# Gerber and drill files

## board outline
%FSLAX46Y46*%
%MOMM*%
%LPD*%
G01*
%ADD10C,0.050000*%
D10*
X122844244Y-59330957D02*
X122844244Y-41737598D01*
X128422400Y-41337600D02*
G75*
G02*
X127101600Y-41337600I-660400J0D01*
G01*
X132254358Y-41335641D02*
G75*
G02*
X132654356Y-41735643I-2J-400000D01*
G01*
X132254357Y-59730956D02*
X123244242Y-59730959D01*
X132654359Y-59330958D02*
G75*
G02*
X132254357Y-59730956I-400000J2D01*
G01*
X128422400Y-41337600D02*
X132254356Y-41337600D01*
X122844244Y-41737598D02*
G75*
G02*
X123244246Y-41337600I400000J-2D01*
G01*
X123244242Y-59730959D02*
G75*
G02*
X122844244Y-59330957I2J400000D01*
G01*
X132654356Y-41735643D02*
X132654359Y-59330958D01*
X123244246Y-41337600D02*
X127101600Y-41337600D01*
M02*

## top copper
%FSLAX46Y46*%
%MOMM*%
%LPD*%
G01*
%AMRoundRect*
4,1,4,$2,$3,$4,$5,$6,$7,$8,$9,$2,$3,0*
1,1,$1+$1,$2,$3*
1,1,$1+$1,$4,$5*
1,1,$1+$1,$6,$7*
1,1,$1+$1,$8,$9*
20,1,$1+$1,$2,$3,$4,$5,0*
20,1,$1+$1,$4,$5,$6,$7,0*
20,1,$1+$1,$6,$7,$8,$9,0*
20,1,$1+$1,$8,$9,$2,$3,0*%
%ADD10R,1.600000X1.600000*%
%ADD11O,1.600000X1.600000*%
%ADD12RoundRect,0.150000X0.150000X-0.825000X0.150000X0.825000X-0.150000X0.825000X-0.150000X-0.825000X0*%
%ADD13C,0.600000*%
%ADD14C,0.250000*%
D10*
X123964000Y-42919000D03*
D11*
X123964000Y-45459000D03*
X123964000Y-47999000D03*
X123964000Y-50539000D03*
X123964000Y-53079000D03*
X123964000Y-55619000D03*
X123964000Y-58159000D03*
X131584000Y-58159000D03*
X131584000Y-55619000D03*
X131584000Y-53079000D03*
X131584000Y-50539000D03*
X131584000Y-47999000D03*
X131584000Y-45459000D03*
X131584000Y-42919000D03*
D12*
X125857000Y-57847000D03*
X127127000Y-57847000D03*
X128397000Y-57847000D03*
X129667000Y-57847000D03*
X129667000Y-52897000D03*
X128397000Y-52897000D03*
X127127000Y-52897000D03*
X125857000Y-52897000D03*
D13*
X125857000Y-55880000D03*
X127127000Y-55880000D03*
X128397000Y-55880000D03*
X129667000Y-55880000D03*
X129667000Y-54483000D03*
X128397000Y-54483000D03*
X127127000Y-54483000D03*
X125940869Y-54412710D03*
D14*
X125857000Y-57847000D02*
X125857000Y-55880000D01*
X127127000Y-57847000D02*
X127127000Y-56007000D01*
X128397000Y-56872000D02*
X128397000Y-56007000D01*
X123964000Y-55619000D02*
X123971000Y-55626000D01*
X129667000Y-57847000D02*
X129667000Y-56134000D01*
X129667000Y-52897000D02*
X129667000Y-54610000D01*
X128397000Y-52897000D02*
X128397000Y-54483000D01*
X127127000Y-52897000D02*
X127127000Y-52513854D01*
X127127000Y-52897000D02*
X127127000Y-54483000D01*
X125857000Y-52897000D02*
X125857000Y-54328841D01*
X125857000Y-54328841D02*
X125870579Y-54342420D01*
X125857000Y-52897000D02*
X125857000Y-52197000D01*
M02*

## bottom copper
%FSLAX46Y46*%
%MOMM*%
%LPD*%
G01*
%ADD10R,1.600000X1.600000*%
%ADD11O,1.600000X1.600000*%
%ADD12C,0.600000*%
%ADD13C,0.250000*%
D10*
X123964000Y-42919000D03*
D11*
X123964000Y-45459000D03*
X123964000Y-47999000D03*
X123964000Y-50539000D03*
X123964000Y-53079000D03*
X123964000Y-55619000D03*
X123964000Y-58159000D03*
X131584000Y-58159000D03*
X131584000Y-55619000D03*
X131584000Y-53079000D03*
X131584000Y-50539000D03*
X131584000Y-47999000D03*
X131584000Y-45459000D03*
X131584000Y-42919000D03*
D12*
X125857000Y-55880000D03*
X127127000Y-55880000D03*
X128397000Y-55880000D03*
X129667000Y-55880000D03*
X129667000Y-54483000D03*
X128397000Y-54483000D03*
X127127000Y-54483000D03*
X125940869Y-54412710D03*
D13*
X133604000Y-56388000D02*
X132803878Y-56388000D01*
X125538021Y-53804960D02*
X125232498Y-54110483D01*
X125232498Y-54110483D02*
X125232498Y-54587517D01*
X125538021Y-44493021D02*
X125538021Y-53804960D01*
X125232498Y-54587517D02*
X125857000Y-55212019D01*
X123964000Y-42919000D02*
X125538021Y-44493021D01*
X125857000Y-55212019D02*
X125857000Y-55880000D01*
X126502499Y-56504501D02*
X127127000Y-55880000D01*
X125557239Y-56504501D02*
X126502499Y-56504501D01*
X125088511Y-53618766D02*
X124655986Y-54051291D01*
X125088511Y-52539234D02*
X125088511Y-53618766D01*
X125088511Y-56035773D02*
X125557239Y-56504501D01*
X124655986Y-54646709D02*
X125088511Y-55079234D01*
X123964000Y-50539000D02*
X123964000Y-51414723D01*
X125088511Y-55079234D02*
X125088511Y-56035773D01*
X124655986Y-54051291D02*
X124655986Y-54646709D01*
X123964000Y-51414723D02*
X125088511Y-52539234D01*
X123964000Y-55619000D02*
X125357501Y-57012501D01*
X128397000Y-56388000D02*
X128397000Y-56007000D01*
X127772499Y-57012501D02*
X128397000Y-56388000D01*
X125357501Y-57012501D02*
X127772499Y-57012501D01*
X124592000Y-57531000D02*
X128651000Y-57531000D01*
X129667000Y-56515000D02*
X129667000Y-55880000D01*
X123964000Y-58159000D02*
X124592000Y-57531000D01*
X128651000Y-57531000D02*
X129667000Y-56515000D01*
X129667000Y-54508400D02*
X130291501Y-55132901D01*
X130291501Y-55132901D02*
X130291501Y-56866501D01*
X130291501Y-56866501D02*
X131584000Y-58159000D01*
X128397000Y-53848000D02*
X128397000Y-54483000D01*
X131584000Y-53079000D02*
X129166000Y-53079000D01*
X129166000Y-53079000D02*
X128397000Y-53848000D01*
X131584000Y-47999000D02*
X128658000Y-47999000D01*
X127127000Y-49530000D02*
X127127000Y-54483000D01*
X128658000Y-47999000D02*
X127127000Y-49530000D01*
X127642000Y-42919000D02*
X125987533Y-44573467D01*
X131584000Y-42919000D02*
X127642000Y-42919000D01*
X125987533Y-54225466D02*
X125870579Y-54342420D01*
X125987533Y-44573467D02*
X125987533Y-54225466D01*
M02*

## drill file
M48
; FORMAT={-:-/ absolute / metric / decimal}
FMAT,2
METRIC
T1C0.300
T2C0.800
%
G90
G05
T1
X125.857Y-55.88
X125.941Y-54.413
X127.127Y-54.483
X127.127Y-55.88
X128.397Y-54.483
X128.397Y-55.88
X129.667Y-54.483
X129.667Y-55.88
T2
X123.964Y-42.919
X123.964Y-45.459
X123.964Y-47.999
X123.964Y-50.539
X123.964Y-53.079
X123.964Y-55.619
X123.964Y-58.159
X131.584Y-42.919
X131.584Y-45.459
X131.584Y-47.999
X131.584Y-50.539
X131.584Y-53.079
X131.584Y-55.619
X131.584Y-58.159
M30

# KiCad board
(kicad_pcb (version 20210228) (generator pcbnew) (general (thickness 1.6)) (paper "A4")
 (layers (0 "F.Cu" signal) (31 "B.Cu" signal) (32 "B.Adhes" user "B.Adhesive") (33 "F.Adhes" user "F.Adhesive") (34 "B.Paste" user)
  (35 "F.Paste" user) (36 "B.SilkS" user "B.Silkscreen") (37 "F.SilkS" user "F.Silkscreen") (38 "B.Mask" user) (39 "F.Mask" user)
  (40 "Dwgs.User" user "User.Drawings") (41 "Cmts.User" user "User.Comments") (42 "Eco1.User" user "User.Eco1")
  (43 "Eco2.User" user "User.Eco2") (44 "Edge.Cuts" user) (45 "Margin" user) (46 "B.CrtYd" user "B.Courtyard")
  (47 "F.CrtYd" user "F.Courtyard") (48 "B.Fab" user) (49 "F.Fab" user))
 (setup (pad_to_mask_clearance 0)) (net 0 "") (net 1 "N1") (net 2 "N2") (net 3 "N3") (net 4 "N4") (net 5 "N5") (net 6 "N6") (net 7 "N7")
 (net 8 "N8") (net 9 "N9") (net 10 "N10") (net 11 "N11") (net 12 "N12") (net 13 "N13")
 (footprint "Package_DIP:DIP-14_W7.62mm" (layer "F.Cu") (at 123.964 42.919)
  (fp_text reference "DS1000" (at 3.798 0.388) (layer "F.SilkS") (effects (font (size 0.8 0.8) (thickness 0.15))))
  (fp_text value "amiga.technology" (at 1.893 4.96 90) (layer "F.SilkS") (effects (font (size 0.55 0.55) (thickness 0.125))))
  (pad "1" thru_hole rect (at 0 0) (locked) (size 1.6 1.6) (drill 0.8) (layers *.Cu *.Mask) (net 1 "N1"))
  (pad "2" thru_hole oval (at 0 2.54) (locked) (size 1.6 1.6) (drill 0.8) (layers *.Cu *.Mask) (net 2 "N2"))
  (pad "3" thru_hole oval (at 0 5.08) (locked) (size 1.6 1.6) (drill 0.8) (layers *.Cu *.Mask) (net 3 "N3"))
  (pad "4" thru_hole oval (at 0 7.62) (locked) (size 1.6 1.6) (drill 0.8) (layers *.Cu *.Mask) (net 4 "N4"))
  (pad "5" thru_hole oval (at 0 10.16) (locked) (size 1.6 1.6) (drill 0.8) (layers *.Cu *.Mask))
  (pad "6" thru_hole oval (at 0 12.7) (locked) (size 1.6 1.6) (drill 0.8) (layers *.Cu *.Mask) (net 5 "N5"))
  (pad "7" thru_hole oval (at 0 15.24) (locked) (size 1.6 1.6) (drill 0.8) (layers *.Cu *.Mask) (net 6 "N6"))
  (pad "8" thru_hole oval (at 7.62 15.24) (locked) (size 1.6 1.6) (drill 0.8) (layers *.Cu *.Mask) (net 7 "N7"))
  (pad "9" thru_hole oval (at 7.62 12.7) (locked) (size 1.6 1.6) (drill 0.8) (layers *.Cu *.Mask) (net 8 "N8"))
  (pad "10" thru_hole oval (at 7.62 10.16) (locked) (size 1.6 1.6) (drill 0.8) (layers *.Cu *.Mask) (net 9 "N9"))
  (pad "11" thru_hole oval (at 7.62 7.62) (locked) (size 1.6 1.6) (drill 0.8) (layers *.Cu *.Mask) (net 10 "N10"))
  (pad "12" thru_hole oval (at 7.62 5.08) (locked) (size 1.6 1.6) (drill 0.8) (layers *.Cu *.Mask) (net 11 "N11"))
  (pad "13" thru_hole oval (at 7.62 2.54) (locked) (size 1.6 1.6) (drill 0.8) (layers *.Cu *.Mask) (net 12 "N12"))
  (pad "14" thru_hole oval (at 7.62 0) (locked) (size 1.6 1.6) (drill 0.8) (layers *.Cu *.Mask) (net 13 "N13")))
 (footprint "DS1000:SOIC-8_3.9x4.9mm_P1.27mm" (layer "F.Cu") (at 127.762 55.372 90)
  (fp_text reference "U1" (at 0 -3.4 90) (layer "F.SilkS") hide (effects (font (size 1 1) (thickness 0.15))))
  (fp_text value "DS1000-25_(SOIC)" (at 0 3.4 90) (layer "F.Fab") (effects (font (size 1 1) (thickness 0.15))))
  (pad "1" smd roundrect (at -2.475 -1.905 90) (locked) (size 1.95 0.6) (layers "F.Cu" "F.Paste" "F.Mask") (roundrect_rratio 0.25)
   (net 1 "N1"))
  (pad "2" smd roundrect (at -2.475 -0.635 90) (locked) (size 1.95 0.6) (layers "F.Cu" "F.Paste" "F.Mask") (roundrect_rratio 0.25)
   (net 4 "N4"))
  (pad "3" smd roundrect (at -2.475 0.635 90) (locked) (size 1.95 0.6) (layers "F.Cu" "F.Paste" "F.Mask") (roundrect_rratio 0.25)
   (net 5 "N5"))
  (pad "4" smd roundrect (at -2.475 1.905 90) (locked) (size 1.95 0.6) (layers "F.Cu" "F.Paste" "F.Mask") (roundrect_rratio 0.25)
   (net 6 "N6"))
  (pad "5" smd roundrect (at 2.475 1.905 90) (locked) (size 1.95 0.6) (layers "F.Cu" "F.Paste" "F.Mask") (roundrect_rratio 0.25)
   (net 7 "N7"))
  (pad "6" smd roundrect (at 2.475 0.635 90) (locked) (size 1.95 0.6) (layers "F.Cu" "F.Paste" "F.Mask") (roundrect_rratio 0.25)
   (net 9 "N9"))
  (pad "7" smd roundrect (at 2.475 -0.635 90) (locked) (size 1.95 0.6) (layers "F.Cu" "F.Paste" "F.Mask") (roundrect_rratio 0.25)
   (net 11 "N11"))
  (pad "8" smd roundrect (at 2.475 -1.905 90) (locked) (size 1.95 0.6) (layers "F.Cu" "F.Paste" "F.Mask") (roundrect_rratio 0.25)
   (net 13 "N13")))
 (gr_line (start 122.844244 59.330957) (end 122.844244 41.737598) (layer "Edge.Cuts") (width 0.05))
 (gr_arc (start 127.762 41.3376) (end 128.4224 41.3376) (angle 180) (layer "Edge.Cuts") (width 0.05))
 (gr_arc (start 132.254356 41.735641) (end 132.654356 41.735643) (angle -90) (layer "Edge.Cuts") (width 0.05))
 (gr_line (start 132.254357 59.730956) (end 123.244242 59.730959) (layer "Edge.Cuts") (width 0.05))
 (gr_arc (start 132.254359 59.330956) (end 132.254357 59.730956) (angle -90) (layer "Edge.Cuts") (width 0.05))
 (gr_line (start 128.4224 41.3376) (end 132.254356 41.3376) (layer "Edge.Cuts") (width 0.05))
 (gr_arc (start 123.244244 41.7376) (end 123.244246 41.3376) (angle -90) (layer "Edge.Cuts") (width 0.05))
 (gr_arc (start 123.244244 59.330959) (end 122.844244 59.330957) (angle -90) (layer "Edge.Cuts") (width 0.05))
 (gr_line (start 132.654356 41.735643) (end 132.654359 59.330958) (layer "Edge.Cuts") (width 0.05))
 (gr_line (start 123.244246 41.3376) (end 127.1016 41.3376) (layer "Edge.Cuts") (width 0.05))
 (segment (start 133.604 56.388) (end 132.803878 56.388) (width 0.25) (layer "B.Cu") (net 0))
 (segment (start 125.857 57.847) (end 125.857 55.88) (width 0.25) (layer "F.Cu") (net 1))
 (via (at 125.857 55.88) (size 0.6) (drill 0.3) (layers "F.Cu" "B.Cu") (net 1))
 (segment (start 125.538021 53.80496) (end 125.232498 54.110483) (width 0.25) (layer "B.Cu") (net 1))
 (segment (start 125.232498 54.110483) (end 125.232498 54.587517) (width 0.25) (layer "B.Cu") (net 1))
 (segment (start 125.538021 44.493021) (end 125.538021 53.80496) (width 0.25) (layer "B.Cu") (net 1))
 (segment (start 125.232498 54.587517) (end 125.857 55.212019) (width 0.25) (layer "B.Cu") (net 1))
 (segment (start 123.964 42.919) (end 125.538021 44.493021) (width 0.25) (layer "B.Cu") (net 1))
 (segment (start 125.857 55.212019) (end 125.857 55.88) (width 0.25) (layer "B.Cu") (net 1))
 (segment (start 127.127 57.847) (end 127.127 56.007) (width 0.25) (layer "F.Cu") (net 4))
 (via (at 127.127 55.88) (size 0.6) (drill 0.3) (layers "F.Cu" "B.Cu") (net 4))
 (segment (start 126.502499 56.504501) (end 127.127 55.88) (width 0.25) (layer "B.Cu") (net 4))
 (segment (start 125.557239 56.504501) (end 126.502499 56.504501) (width 0.25) (layer "B.Cu") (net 4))
 (segment (start 125.088511 53.618766) (end 124.655986 54.051291) (width 0.25) (layer "B.Cu") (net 4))
 (segment (start 125.088511 52.539234) (end 125.088511 53.618766) (width 0.25) (layer "B.Cu") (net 4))
 (segment (start 125.088511 56.035773) (end 125.557239 56.504501) (width 0.25) (layer "B.Cu") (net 4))
 (segment (start 124.655986 54.646709) (end 125.088511 55.079234) (width 0.25) (layer "B.Cu") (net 4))
 (segment (start 123.964 50.539) (end 123.964 51.414723) (width 0.25) (layer "B.Cu") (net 4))
 (segment (start 125.088511 55.079234) (end 125.088511 56.035773) (width 0.25) (layer "B.Cu") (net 4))
 (segment (start 124.655986 54.051291) (end 124.655986 54.646709) (width 0.25) (layer "B.Cu") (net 4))
 (segment (start 123.964 51.414723) (end 125.088511 52.539234) (width 0.25) (layer "B.Cu") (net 4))
 (segment (start 128.397 56.872) (end 128.397 56.007) (width 0.25) (layer "F.Cu") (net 5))
 (segment (start 123.964 55.619) (end 123.971 55.626) (width 0.25) (layer "F.Cu") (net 5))
 (via (at 128.397 55.88) (size 0.6) (drill 0.3) (layers "F.Cu" "B.Cu") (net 5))
 (segment (start 123.964 55.619) (end 125.357501 57.012501) (width 0.25) (layer "B.Cu") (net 5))
 (segment (start 128.397 56.388) (end 128.397 56.007) (width 0.25) (layer "B.Cu") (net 5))
 (segment (start 127.772499 57.012501) (end 128.397 56.388) (width 0.25) (layer "B.Cu") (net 5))
 (segment (start 125.357501 57.012501) (end 127.772499 57.012501) (width 0.25) (layer "B.Cu") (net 5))
 (segment (start 129.667 57.847) (end 129.667 56.134) (width 0.25) (layer "F.Cu") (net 6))
 (via (at 129.667 55.88) (size 0.6) (drill 0.3) (layers "F.Cu" "B.Cu") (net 6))
 (segment (start 124.592 57.531) (end 128.651 57.531) (width 0.25) (layer "B.Cu") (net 6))
 (segment (start 129.667 56.515) (end 129.667 55.88) (width 0.25) (layer "B.Cu") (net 6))
 (segment (start 123.964 58.159) (end 124.592 57.531) (width 0.25) (layer "B.Cu") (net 6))
 (segment (start 128.651 57.531) (end 129.667 56.515) (width 0.25) (layer "B.Cu") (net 6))
 (segment (start 129.667 52.897) (end 129.667 54.61) (width 0.25) (layer "F.Cu") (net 7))
 (via (at 129.667 54.483) (size 0.6) (drill 0.3) (layers "F.Cu" "B.Cu") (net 7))
 (segment (start 129.667 54.5084) (end 130.291501 55.132901) (width 0.25) (layer "B.Cu") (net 7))
 (segment (start 130.291501 55.132901) (end 130.291501 56.866501) (width 0.25) (layer "B.Cu") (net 7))
 (segment (start 130.291501 56.866501) (end 131.584 58.159) (width 0.25) (layer "B.Cu") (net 7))
 (segment (start 128.397 52.897) (end 128.397 54.483) (width 0.25) (layer "F.Cu") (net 9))
 (via (at 128.397 54.483) (size 0.6) (drill 0.3) (layers "F.Cu" "B.Cu") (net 9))
 (segment (start 128.397 53.848) (end 128.397 54.483) (width 0.25) (layer "B.Cu") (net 9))
 (segment (start 131.584 53.079) (end 129.166 53.079) (width 0.25) (layer "B.Cu") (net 9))
 (segment (start 129.166 53.079) (end 128.397 53.848) (width 0.25) (layer "B.Cu") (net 9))
 (segment (start 127.127 52.897) (end 127.127 52.513854) (width 0.25) (layer "F.Cu") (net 11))
 (segment (start 127.127 52.897) (end 127.127 54.483) (width 0.25) (layer "F.Cu") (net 11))
 (via (at 127.127 54.483) (size 0.6) (drill 0.3) (layers "F.Cu" "B.Cu") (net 11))
 (segment (start 131.584 47.999) (end 128.658 47.999) (width 0.25) (layer "B.Cu") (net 11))
 (segment (start 127.127 49.53) (end 127.127 54.483) (width 0.25) (layer "B.Cu") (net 11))
 (segment (start 128.658 47.999) (end 127.127 49.53) (width 0.25) (layer "B.Cu") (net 11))
 (segment (start 125.857 52.897) (end 125.857 54.328841) (width 0.25) (layer "F.Cu") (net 13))
 (segment (start 125.857 54.328841) (end 125.870579 54.34242) (width 0.25) (layer "F.Cu") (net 13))
 (segment (start 125.857 52.897) (end 125.857 52.197) (width 0.25) (layer "F.Cu") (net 13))
 (via (at 125.940869 54.41271) (size 0.6) (drill 0.3) (layers "F.Cu" "B.Cu") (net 13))
 (segment (start 127.642 42.919) (end 125.987533 44.573467) (width 0.25) (layer "B.Cu") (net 13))
 (segment (start 131.584 42.919) (end 127.642 42.919) (width 0.25) (layer "B.Cu") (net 13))
 (segment (start 125.987533 54.225466) (end 125.870579 54.34242) (width 0.25) (layer "B.Cu") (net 13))
 (segment (start 125.987533 44.573467) (end 125.987533 54.225466) (width 0.25) (layer "B.Cu") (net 13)))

